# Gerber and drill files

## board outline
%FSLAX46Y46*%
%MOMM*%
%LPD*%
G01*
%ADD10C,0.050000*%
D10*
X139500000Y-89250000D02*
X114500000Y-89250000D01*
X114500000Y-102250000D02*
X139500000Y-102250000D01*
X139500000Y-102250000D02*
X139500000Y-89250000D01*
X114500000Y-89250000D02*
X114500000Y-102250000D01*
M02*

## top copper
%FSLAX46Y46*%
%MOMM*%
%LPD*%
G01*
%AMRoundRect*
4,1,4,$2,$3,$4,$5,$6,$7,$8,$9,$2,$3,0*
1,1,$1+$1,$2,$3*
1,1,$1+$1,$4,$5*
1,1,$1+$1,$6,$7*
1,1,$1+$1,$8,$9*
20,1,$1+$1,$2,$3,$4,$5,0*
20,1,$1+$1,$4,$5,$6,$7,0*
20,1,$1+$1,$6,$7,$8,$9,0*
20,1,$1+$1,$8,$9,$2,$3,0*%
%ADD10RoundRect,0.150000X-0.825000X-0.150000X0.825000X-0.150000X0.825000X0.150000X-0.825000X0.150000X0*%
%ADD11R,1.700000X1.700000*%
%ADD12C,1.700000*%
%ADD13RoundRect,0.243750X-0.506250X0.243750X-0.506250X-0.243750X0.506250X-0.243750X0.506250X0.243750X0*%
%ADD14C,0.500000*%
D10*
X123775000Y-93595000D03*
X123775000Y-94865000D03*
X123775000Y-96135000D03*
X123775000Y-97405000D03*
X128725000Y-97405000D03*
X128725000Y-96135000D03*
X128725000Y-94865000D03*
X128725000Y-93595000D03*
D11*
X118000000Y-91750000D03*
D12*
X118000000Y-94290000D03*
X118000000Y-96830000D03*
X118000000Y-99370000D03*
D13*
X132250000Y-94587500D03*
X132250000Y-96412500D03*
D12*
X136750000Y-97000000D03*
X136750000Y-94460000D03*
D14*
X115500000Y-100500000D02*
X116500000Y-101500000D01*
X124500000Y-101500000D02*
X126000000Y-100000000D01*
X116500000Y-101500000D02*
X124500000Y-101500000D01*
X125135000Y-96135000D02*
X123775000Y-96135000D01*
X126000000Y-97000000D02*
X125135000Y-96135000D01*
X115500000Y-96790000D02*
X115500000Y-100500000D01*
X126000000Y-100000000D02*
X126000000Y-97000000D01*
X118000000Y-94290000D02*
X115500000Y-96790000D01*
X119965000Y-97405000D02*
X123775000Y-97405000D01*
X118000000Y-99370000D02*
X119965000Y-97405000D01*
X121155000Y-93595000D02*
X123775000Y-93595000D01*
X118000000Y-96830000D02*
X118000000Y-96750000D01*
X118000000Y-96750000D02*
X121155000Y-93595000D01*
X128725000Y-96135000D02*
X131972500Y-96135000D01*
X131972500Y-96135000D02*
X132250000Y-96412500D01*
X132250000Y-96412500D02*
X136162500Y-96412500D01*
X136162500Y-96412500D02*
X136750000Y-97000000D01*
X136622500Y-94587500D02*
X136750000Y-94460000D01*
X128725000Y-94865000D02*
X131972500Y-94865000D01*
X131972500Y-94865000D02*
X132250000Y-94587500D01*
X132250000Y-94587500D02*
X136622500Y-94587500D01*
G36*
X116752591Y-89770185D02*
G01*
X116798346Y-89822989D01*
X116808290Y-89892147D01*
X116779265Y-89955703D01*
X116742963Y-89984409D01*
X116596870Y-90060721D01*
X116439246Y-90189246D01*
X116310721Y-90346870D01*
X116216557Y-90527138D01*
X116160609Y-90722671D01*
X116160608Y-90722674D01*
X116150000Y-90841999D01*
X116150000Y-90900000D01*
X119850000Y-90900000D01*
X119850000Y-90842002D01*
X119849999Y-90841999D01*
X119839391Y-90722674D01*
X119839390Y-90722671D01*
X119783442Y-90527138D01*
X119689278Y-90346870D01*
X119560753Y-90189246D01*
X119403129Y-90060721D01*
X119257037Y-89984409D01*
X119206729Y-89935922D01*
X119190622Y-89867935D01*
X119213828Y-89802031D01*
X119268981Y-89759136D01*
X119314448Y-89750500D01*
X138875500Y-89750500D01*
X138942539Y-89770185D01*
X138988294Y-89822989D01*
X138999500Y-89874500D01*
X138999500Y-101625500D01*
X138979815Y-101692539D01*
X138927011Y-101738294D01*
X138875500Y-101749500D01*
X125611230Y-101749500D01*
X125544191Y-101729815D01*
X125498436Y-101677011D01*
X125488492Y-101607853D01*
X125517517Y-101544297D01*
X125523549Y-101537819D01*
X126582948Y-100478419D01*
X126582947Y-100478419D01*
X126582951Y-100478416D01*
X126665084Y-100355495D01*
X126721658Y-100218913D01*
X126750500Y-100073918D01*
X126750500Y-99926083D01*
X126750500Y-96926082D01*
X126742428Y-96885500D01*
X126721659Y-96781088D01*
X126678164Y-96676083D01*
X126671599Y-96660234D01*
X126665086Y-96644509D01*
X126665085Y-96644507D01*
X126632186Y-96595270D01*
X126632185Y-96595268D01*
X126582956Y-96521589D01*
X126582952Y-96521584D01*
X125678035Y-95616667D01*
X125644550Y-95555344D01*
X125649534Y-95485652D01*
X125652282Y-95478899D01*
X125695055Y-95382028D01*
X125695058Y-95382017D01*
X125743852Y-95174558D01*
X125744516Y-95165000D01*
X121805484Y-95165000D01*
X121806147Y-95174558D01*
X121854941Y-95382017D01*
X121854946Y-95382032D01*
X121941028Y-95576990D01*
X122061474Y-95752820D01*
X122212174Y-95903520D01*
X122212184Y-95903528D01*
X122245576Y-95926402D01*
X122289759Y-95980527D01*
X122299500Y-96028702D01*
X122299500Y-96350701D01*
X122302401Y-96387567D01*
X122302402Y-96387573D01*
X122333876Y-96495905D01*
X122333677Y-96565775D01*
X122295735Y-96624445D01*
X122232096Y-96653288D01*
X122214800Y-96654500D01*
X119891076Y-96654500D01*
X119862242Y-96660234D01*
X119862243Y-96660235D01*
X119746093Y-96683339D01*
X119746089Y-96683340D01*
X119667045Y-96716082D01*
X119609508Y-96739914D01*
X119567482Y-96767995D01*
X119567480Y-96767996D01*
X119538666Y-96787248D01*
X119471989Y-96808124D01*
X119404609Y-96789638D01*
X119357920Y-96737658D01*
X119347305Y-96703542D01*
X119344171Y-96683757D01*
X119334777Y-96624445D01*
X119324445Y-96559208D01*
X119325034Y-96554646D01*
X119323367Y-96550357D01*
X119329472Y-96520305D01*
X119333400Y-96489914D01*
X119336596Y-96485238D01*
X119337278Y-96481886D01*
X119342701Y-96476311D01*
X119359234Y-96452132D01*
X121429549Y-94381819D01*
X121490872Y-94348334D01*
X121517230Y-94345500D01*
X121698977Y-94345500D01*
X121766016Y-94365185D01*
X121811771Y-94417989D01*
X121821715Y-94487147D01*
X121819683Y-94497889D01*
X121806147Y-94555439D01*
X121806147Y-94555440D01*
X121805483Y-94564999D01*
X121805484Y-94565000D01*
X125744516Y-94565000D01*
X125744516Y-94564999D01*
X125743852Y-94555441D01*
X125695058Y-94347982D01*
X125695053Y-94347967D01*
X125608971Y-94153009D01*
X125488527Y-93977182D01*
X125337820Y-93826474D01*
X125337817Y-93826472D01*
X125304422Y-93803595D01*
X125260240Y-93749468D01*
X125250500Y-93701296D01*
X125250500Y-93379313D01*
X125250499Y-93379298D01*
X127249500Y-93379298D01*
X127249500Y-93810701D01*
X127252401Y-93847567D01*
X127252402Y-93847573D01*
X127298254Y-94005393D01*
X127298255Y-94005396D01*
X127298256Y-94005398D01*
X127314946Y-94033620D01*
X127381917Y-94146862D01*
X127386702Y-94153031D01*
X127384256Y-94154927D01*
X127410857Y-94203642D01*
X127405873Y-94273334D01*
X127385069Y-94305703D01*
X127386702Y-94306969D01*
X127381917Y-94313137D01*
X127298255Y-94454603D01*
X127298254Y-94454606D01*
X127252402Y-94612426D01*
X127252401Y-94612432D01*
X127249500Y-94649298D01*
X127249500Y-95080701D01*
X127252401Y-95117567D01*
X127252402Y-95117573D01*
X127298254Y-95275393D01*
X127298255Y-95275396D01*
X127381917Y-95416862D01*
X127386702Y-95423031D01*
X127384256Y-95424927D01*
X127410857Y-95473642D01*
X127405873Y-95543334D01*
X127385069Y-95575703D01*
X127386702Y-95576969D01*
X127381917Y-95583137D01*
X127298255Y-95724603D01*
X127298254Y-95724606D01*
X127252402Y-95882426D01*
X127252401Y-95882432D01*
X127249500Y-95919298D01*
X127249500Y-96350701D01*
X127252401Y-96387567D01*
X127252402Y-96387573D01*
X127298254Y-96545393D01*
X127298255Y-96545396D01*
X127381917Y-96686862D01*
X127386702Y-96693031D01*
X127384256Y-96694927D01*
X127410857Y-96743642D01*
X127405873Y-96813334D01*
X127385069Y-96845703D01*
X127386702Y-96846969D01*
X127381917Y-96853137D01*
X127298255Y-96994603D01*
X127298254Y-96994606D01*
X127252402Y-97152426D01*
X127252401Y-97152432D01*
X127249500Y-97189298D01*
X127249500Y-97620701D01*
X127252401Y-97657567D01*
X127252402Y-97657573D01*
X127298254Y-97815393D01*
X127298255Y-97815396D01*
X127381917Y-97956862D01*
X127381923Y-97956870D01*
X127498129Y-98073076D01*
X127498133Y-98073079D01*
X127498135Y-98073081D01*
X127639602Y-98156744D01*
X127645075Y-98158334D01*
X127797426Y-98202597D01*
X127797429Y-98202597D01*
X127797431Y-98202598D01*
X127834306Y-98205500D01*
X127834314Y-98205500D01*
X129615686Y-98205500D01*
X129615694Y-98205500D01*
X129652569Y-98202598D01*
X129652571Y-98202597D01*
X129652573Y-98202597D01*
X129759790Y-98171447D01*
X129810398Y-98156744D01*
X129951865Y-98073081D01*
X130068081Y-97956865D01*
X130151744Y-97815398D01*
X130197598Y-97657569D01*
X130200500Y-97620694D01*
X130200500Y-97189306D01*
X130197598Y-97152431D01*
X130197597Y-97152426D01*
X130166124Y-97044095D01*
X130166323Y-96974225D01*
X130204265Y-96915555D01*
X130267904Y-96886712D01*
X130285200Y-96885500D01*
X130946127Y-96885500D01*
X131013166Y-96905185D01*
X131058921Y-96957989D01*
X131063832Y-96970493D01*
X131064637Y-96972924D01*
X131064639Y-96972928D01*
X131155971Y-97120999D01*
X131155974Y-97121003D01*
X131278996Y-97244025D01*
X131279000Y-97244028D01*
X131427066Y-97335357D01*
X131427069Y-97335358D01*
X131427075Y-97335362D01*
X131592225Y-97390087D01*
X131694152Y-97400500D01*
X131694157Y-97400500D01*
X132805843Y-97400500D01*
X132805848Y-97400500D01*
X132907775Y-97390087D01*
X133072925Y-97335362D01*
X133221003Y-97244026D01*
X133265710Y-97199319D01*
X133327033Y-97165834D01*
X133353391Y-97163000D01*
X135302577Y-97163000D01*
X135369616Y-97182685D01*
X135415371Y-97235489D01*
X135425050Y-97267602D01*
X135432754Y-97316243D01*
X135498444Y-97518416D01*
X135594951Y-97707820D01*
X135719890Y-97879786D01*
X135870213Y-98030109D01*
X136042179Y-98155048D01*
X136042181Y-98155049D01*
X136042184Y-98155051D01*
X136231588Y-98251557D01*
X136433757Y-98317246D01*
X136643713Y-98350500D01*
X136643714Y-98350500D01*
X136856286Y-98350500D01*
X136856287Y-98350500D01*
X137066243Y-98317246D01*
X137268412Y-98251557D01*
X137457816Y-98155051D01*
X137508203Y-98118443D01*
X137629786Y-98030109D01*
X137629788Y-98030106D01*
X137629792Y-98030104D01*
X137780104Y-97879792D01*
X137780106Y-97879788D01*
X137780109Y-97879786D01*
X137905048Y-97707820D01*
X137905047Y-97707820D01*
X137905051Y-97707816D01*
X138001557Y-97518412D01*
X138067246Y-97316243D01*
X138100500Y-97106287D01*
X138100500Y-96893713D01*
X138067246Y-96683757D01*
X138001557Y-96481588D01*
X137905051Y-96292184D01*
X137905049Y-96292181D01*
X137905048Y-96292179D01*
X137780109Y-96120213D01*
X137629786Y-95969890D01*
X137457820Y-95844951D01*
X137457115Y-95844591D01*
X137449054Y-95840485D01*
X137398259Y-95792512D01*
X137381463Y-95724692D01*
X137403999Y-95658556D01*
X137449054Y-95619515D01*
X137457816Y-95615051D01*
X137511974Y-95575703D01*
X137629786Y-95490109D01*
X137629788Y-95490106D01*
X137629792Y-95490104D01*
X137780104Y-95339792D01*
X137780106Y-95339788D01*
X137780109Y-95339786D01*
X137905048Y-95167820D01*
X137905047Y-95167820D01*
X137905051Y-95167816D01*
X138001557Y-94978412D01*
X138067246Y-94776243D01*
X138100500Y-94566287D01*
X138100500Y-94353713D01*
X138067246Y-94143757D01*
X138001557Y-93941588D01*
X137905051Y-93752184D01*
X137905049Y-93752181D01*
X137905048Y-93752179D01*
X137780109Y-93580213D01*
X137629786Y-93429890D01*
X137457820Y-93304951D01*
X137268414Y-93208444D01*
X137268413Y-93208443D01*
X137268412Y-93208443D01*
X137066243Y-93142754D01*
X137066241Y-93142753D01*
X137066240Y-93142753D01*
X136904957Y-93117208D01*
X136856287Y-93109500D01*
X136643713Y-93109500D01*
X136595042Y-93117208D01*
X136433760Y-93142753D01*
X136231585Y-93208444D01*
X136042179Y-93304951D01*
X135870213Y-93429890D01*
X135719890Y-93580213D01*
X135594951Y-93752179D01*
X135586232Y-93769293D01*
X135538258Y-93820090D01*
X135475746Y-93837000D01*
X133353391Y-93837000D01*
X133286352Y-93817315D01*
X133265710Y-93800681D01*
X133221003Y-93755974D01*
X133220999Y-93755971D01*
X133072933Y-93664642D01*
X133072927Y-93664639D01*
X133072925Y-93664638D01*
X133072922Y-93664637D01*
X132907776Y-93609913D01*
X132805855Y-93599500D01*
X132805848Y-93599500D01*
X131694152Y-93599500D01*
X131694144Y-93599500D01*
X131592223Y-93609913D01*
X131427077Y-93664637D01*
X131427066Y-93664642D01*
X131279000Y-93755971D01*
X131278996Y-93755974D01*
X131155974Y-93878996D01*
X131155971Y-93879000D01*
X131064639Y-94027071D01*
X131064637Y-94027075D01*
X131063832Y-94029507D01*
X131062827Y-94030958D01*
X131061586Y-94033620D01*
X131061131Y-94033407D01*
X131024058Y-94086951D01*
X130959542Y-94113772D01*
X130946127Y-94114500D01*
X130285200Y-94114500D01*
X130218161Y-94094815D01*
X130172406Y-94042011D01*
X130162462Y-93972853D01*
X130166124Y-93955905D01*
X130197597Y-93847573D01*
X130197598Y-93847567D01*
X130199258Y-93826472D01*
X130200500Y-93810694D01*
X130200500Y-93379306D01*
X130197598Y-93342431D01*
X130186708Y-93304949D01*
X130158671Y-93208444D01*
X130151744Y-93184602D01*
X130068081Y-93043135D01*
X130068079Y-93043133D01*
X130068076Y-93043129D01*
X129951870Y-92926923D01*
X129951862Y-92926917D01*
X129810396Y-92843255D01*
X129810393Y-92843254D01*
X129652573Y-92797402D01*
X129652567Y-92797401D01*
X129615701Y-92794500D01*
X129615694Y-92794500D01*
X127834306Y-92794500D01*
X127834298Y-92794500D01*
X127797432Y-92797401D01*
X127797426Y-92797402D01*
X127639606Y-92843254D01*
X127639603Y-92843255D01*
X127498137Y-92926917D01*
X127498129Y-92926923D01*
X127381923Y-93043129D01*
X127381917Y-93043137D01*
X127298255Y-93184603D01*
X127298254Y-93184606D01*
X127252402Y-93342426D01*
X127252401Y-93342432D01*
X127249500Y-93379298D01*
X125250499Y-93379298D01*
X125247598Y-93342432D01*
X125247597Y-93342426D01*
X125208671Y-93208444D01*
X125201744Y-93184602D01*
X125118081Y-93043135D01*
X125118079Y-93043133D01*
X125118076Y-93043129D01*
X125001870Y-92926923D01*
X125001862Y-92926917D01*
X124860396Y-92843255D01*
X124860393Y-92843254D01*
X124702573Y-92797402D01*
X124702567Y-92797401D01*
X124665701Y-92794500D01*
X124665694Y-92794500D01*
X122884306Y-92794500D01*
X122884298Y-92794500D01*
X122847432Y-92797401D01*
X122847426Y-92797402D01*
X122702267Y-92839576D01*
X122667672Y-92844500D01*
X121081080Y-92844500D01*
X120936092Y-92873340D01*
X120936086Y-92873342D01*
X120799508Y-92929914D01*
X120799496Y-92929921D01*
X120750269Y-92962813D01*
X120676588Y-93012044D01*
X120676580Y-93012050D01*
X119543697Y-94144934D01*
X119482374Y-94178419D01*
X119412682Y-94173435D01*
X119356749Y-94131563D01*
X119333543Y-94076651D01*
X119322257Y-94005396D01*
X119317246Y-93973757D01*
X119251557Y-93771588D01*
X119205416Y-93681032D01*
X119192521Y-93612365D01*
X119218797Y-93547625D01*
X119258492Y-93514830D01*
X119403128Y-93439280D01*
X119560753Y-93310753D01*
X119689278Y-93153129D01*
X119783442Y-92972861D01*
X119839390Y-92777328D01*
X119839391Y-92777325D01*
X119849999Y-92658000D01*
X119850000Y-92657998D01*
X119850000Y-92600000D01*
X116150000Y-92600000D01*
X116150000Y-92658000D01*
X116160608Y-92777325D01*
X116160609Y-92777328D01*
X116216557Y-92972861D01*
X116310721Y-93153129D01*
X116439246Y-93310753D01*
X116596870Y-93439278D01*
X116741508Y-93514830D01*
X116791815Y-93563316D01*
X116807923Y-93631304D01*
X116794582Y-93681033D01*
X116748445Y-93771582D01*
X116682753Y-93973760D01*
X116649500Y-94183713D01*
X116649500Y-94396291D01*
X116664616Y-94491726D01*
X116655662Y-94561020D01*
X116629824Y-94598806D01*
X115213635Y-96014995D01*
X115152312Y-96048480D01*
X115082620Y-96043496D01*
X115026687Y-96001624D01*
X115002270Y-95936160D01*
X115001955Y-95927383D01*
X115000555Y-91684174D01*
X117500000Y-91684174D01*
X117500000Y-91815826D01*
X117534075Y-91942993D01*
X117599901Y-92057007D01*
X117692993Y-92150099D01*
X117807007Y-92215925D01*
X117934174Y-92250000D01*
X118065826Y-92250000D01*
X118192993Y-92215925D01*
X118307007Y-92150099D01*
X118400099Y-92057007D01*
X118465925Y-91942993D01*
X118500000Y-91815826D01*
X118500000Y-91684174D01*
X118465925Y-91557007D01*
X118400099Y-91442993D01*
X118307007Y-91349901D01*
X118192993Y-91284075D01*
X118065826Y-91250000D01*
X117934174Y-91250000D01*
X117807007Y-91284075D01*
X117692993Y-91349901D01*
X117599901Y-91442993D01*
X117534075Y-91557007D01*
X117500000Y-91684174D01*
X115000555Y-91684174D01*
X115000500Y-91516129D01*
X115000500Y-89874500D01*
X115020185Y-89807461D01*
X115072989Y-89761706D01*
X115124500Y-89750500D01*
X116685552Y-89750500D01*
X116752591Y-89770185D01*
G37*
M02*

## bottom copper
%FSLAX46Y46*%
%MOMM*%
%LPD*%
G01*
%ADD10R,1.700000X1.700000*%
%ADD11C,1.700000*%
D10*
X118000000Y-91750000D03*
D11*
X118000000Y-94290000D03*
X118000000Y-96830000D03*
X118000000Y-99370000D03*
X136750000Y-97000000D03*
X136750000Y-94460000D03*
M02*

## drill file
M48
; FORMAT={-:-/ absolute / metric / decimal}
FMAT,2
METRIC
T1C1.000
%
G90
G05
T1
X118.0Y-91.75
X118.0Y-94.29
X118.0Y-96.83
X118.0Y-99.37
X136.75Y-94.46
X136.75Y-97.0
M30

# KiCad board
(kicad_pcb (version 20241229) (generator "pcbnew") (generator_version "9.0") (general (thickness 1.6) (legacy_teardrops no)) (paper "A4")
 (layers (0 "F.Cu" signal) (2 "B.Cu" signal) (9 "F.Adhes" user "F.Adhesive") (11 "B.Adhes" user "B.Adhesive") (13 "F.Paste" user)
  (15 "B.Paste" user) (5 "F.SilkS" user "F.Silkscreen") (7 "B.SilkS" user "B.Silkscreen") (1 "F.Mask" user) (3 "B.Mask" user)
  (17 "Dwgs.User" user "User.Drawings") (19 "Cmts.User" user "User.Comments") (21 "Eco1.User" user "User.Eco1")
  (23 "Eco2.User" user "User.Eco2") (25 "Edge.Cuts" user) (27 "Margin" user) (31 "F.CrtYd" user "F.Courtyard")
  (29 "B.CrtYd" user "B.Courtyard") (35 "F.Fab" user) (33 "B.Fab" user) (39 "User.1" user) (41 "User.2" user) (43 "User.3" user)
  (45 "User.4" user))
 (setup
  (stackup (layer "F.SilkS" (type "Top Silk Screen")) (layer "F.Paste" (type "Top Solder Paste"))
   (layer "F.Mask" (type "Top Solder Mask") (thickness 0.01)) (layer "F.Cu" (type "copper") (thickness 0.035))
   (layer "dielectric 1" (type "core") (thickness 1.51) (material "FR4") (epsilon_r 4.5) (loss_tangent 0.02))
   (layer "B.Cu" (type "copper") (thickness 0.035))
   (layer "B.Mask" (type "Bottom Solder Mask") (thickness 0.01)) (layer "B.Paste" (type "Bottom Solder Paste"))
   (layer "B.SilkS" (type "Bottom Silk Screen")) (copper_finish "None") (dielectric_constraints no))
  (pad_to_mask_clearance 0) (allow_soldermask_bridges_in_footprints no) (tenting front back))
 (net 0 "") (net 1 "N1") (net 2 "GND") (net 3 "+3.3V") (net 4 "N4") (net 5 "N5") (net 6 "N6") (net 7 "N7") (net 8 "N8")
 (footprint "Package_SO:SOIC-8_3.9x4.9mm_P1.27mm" (layer "F.Cu") (at 126.25 95.5)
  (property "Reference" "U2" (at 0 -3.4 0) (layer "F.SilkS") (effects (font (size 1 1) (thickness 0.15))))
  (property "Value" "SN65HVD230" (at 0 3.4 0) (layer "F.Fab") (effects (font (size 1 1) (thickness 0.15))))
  (pad "1" smd roundrect (at -2.475 -1.905) (size 1.95 0.6) (layers "F.Cu" "F.Mask" "F.Paste") (roundrect_rratio 0.25) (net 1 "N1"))
  (pad "2" smd roundrect (at -2.475 -0.635) (size 1.95 0.6) (layers "F.Cu" "F.Mask" "F.Paste") (roundrect_rratio 0.25) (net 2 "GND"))
  (pad "3" smd roundrect (at -2.475 0.635) (size 1.95 0.6) (layers "F.Cu" "F.Mask" "F.Paste") (roundrect_rratio 0.25) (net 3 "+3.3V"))
  (pad "4" smd roundrect (at -2.475 1.905) (size 1.95 0.6) (layers "F.Cu" "F.Mask" "F.Paste") (roundrect_rratio 0.25) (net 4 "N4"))
  (pad "5" smd roundrect (at 2.475 1.905) (size 1.95 0.6) (layers "F.Cu" "F.Mask" "F.Paste") (roundrect_rratio 0.25) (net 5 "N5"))
  (pad "6" smd roundrect (at 2.475 0.635) (size 1.95 0.6) (layers "F.Cu" "F.Mask" "F.Paste") (roundrect_rratio 0.25) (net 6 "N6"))
  (pad "7" smd roundrect (at 2.475 -0.635) (size 1.95 0.6) (layers "F.Cu" "F.Mask" "F.Paste") (roundrect_rratio 0.25) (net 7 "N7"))
  (pad "8" smd roundrect (at 2.475 -1.905) (size 1.95 0.6) (layers "F.Cu" "F.Mask" "F.Paste") (roundrect_rratio 0.25) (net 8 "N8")))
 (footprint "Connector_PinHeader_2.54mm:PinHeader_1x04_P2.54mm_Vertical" (layer "F.Cu") (at 118 91.75)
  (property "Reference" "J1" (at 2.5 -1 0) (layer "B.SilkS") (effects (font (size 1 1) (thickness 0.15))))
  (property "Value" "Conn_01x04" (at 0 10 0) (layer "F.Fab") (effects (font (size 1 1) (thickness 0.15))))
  (pad "1" thru_hole rect (at 0 0) (size 1.7 1.7) (drill 1) (layers "*.Cu" "*.Mask") (remove_unused_layers no) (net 2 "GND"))
  (pad "2" thru_hole circle (at 0 2.54) (size 1.7 1.7) (drill 1) (layers "*.Cu" "*.Mask") (remove_unused_layers no) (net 3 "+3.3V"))
  (pad "3" thru_hole circle (at 0 5.08) (size 1.7 1.7) (drill 1) (layers "*.Cu" "*.Mask") (remove_unused_layers no) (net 1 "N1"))
  (pad "4" thru_hole circle (at 0 7.62) (size 1.7 1.7) (drill 1) (layers "*.Cu" "*.Mask") (remove_unused_layers no) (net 4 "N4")))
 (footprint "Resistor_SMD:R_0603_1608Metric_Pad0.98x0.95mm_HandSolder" (layer "F.Cu") (at 132.25 95.5 -90)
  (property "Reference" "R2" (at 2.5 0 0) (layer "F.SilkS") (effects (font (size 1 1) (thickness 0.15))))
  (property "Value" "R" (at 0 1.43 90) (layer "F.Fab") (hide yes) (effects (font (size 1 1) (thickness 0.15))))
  (pad "1" smd roundrect (at -0.9125 0 270) (size 0.975 1.5) (layers "F.Cu" "F.Mask" "F.Paste") (roundrect_rratio 0.25) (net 7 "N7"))
  (pad "2" smd roundrect (at 0.9125 0 270) (size 0.975 1.5) (layers "F.Cu" "F.Mask" "F.Paste") (roundrect_rratio 0.25) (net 6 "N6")))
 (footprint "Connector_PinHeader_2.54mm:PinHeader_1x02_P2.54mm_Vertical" (layer "F.Cu") (at 136.75 97 180)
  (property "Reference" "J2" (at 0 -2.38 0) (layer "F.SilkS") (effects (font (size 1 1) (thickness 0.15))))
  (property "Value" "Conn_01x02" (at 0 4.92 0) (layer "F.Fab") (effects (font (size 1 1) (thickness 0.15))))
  (pad "1" thru_hole circle (at 0 0 180) (size 1.7 1.7) (drill 1) (layers "*.Cu" "*.Mask") (remove_unused_layers no) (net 6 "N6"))
  (pad "2" thru_hole circle (at 0 2.54 180) (size 1.7 1.7) (drill 1) (layers "*.Cu" "*.Mask") (remove_unused_layers no) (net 7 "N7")))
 (gr_line (start 139.5 89.25) (end 114.5 89.25) (stroke (width 0.05) (type default)) (layer "Edge.Cuts"))
 (gr_line (start 114.5 102.25) (end 139.5 102.25) (stroke (width 0.05) (type default)) (layer "Edge.Cuts"))
 (gr_line (start 139.5 102.25) (end 139.5 89.25) (stroke (width 0.05) (type default)) (layer "Edge.Cuts"))
 (gr_line (start 114.5 89.25) (end 114.5 102.25) (stroke (width 0.05) (type default)) (layer "Edge.Cuts"))
 (segment (start 115.5 100.5) (end 116.5 101.5) (width 0.5) (layer "F.Cu") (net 3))
 (segment (start 124.5 101.5) (end 126 100) (width 0.5) (layer "F.Cu") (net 3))
 (segment (start 116.5 101.5) (end 124.5 101.5) (width 0.5) (layer "F.Cu") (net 3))
 (segment (start 125.135 96.135) (end 123.775 96.135) (width 0.5) (layer "F.Cu") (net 3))
 (segment (start 126 97) (end 125.135 96.135) (width 0.5) (layer "F.Cu") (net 3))
 (segment (start 115.5 96.79) (end 115.5 100.5) (width 0.5) (layer "F.Cu") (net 3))
 (segment (start 126 100) (end 126 97) (width 0.5) (layer "F.Cu") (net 3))
 (segment (start 118 94.29) (end 115.5 96.79) (width 0.5) (layer "F.Cu") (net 3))
 (segment (start 119.965 97.405) (end 123.775 97.405) (width 0.5) (layer "F.Cu") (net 4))
 (segment (start 118 99.37) (end 119.965 97.405) (width 0.5) (layer "F.Cu") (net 4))
 (segment (start 121.155 93.595) (end 123.775 93.595) (width 0.5) (layer "F.Cu") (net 1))
 (segment (start 118 96.83) (end 118 96.75) (width 0.5) (layer "F.Cu") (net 1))
 (segment (start 118 96.75) (end 121.155 93.595) (width 0.5) (layer "F.Cu") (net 1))
 (segment (start 128.725 96.135) (end 131.9725 96.135) (width 0.5) (layer "F.Cu") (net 6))
 (segment (start 131.9725 96.135) (end 132.25 96.4125) (width 0.5) (layer "F.Cu") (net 6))
 (segment (start 132.25 96.4125) (end 136.1625 96.4125) (width 0.5) (layer "F.Cu") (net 6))
 (segment (start 136.1625 96.4125) (end 136.75 97) (width 0.5) (layer "F.Cu") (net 6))
 (segment (start 136.6225 94.5875) (end 136.75 94.46) (width 0.5) (layer "F.Cu") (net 7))
 (segment (start 128.725 94.865) (end 131.9725 94.865) (width 0.5) (layer "F.Cu") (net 7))
 (segment (start 131.9725 94.865) (end 132.25 94.5875) (width 0.5) (layer "F.Cu") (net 7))
 (segment (start 132.25 94.5875) (end 136.6225 94.5875) (width 0.5) (layer "F.Cu") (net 7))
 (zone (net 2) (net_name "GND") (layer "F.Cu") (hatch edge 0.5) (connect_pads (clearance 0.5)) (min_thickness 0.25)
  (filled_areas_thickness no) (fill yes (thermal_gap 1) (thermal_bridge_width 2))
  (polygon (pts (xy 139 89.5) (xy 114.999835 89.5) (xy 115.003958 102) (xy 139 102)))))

